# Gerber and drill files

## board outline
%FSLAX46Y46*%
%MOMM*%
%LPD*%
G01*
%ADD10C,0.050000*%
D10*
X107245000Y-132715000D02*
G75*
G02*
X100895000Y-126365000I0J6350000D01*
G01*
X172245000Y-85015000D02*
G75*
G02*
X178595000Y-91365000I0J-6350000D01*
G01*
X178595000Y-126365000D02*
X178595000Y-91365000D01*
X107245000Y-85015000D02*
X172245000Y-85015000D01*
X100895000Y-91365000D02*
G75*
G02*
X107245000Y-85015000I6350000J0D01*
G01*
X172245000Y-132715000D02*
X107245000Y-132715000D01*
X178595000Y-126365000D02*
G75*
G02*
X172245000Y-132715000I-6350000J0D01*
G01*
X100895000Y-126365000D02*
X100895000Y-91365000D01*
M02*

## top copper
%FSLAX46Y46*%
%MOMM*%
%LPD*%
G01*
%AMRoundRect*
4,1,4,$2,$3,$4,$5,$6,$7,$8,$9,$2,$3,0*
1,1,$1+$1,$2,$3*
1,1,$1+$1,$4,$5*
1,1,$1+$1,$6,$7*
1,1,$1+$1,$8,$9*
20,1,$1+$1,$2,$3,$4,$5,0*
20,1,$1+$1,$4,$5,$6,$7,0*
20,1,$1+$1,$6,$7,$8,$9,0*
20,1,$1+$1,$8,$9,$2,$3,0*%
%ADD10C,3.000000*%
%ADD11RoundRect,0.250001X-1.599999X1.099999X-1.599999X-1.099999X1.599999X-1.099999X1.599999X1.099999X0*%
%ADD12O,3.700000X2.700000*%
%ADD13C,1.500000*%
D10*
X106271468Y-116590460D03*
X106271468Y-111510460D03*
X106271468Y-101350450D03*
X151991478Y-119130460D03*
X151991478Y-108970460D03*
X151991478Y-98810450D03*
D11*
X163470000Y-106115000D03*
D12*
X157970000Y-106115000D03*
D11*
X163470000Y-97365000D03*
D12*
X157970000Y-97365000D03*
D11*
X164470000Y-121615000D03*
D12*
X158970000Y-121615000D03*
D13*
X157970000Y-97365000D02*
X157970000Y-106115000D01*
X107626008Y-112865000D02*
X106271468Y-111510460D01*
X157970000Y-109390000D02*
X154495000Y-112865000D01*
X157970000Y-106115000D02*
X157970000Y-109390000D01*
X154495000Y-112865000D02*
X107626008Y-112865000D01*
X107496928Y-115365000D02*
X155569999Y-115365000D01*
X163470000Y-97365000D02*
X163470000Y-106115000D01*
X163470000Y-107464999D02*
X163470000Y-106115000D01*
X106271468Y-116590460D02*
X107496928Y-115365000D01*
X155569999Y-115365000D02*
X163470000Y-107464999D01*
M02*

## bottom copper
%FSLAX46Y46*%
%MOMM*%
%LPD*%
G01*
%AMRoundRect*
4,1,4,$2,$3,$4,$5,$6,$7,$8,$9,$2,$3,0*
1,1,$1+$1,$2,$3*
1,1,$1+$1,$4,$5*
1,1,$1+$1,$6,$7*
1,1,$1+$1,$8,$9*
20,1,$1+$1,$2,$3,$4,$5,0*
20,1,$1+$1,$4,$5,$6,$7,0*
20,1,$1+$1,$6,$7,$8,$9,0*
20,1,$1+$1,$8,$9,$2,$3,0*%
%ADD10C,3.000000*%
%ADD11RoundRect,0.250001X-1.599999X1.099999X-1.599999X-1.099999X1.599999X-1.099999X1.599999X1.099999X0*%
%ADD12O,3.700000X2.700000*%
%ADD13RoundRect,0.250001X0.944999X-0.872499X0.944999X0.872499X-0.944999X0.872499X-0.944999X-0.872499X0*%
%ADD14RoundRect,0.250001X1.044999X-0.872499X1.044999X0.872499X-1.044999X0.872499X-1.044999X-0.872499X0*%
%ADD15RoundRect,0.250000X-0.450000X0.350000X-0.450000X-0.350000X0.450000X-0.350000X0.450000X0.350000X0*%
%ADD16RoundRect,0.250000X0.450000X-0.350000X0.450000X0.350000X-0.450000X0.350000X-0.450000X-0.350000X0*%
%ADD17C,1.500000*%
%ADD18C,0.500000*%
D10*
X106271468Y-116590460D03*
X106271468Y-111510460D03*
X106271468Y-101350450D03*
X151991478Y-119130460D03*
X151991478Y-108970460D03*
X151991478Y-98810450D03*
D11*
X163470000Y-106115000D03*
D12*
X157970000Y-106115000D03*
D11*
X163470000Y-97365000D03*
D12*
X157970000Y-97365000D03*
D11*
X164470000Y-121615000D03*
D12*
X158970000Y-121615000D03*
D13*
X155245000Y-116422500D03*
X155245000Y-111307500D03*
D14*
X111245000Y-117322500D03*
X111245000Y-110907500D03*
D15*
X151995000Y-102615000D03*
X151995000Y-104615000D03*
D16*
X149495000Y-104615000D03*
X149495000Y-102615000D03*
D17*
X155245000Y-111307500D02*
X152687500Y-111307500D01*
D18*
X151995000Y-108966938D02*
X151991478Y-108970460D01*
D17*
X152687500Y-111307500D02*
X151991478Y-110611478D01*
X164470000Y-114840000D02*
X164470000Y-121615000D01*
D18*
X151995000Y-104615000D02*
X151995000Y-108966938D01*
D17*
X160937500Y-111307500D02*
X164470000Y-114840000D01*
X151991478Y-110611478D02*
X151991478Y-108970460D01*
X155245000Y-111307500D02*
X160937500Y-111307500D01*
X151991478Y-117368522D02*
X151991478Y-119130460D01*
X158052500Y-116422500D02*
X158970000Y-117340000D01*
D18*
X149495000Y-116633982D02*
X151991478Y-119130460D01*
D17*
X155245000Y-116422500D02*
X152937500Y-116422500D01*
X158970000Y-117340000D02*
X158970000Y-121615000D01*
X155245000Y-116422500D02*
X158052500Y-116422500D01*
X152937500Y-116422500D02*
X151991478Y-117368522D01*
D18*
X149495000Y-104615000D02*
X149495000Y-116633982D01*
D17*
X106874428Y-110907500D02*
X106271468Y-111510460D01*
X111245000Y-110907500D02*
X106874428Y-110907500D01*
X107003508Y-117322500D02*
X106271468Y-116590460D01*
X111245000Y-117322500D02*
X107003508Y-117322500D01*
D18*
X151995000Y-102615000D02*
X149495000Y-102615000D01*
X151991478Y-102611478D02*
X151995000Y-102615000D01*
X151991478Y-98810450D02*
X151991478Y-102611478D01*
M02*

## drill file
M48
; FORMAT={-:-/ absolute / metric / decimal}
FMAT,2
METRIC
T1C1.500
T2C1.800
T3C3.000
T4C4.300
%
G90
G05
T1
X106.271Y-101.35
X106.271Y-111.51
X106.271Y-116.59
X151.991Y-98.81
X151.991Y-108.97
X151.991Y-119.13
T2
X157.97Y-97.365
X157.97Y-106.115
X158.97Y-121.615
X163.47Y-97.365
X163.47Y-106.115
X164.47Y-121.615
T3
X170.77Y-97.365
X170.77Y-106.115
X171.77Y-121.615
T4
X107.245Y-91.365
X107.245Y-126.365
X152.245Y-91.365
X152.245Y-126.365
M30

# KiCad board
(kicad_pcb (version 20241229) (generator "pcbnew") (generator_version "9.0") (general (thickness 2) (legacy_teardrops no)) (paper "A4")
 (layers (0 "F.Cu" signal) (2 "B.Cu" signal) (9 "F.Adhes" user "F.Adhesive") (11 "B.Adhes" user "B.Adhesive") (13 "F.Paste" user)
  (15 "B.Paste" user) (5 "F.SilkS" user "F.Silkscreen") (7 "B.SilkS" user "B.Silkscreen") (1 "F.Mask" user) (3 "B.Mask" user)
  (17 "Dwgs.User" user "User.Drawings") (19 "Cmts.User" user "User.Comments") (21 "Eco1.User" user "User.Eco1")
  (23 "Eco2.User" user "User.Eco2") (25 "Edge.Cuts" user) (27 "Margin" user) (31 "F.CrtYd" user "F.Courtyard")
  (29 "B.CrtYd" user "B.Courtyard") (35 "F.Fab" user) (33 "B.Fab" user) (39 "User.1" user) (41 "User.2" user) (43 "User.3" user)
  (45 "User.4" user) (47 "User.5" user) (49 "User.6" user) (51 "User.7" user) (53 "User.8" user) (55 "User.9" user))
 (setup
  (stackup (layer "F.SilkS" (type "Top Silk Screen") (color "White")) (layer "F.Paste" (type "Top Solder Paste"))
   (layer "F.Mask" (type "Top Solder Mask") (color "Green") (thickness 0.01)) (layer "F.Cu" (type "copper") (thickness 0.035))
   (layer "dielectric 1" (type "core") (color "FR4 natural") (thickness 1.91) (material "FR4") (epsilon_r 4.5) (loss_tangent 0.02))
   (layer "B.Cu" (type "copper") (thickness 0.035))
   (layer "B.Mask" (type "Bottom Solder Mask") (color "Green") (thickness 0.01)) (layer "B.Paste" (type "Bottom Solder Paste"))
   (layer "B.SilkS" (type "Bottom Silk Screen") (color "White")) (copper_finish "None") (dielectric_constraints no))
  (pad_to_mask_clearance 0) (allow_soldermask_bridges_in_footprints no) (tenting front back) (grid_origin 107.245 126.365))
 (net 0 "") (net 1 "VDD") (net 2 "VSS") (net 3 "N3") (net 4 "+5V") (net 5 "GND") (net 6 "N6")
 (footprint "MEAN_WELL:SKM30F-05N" (layer "F.Cu") (at 129.185753 95.93234)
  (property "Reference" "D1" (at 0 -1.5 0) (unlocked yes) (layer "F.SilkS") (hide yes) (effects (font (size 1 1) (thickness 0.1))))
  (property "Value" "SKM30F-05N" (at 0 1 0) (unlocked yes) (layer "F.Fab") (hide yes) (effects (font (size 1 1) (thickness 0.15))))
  (pad "1" thru_hole circle (at -22.914285 20.65812 180) (size 3 3) (drill 1.5) (layers "*.Cu" "*.Mask") (remove_unused_layers no)
   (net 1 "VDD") (thermal_bridge_angle 90))
  (pad "2" thru_hole circle (at -22.914285 15.57812 180) (size 3 3) (drill 1.5) (layers "*.Cu" "*.Mask") (remove_unused_layers no)
   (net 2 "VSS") (thermal_bridge_angle 90))
  (pad "3" thru_hole circle (at -22.914285 5.41811 180) (size 3 3) (drill 1.5) (layers "*.Cu" "*.Mask") (remove_unused_layers no)
   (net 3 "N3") (thermal_bridge_angle 90))
  (pad "4" thru_hole circle (at 22.805725 23.19812 180) (size 3 3) (drill 1.5) (layers "*.Cu" "*.Mask") (remove_unused_layers no)
   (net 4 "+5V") (thermal_bridge_angle 90))
  (pad "5" thru_hole circle (at 22.805725 13.03812 180) (size 3 3) (drill 1.5) (layers "*.Cu" "*.Mask") (remove_unused_layers no)
   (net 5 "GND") (thermal_bridge_angle 90))
  (pad "6" thru_hole circle (at 22.805725 2.87811 180) (size 3 3) (drill 1.5) (layers "*.Cu" "*.Mask") (remove_unused_layers no)
   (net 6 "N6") (thermal_bridge_angle 90)))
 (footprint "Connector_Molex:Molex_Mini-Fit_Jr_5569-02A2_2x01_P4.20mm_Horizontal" (layer "F.Cu") (at 163.47 106.115 -90)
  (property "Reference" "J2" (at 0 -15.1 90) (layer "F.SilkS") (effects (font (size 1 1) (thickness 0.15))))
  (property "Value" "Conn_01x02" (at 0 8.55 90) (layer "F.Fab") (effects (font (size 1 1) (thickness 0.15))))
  (pad "" np_thru_hole circle (at 0 -7.3 270) (size 3 3) (drill 3) (layers "*.Cu" "*.Mask"))
  (pad "1" thru_hole roundrect (at 0 0 270) (size 2.7 3.7) (drill 1.8) (layers "*.Cu" "*.Mask") (remove_unused_layers no)
   (roundrect_rratio 0.092593) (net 1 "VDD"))
  (pad "2" thru_hole oval (at 0 5.5 270) (size 2.7 3.7) (drill 1.8) (layers "*.Cu" "*.Mask") (remove_unused_layers no) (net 2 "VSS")))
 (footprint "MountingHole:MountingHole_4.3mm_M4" (layer "F.Cu") (at 107.245 126.365)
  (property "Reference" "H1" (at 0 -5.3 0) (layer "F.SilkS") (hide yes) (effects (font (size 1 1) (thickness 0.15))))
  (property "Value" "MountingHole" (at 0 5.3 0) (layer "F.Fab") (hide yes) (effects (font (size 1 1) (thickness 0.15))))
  (pad "" np_thru_hole circle (at 0 0) (size 4.3 4.3) (drill 4.3) (layers "*.Cu" "*.Mask")))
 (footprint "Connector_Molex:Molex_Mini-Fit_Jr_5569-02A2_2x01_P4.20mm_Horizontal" (layer "F.Cu") (at 163.47 97.365 -90)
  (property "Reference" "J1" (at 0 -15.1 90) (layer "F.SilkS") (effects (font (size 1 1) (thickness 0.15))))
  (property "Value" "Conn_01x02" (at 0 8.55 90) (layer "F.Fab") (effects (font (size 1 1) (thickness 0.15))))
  (pad "" np_thru_hole circle (at 0 -7.3 270) (size 3 3) (drill 3) (layers "*.Cu" "*.Mask"))
  (pad "1" thru_hole roundrect (at 0 0 270) (size 2.7 3.7) (drill 1.8) (layers "*.Cu" "*.Mask") (remove_unused_layers no)
   (roundrect_rratio 0.092593) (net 1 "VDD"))
  (pad "2" thru_hole oval (at 0 5.5 270) (size 2.7 3.7) (drill 1.8) (layers "*.Cu" "*.Mask") (remove_unused_layers no) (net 2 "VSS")))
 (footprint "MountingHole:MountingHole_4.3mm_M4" (layer "F.Cu") (at 107.245 91.365)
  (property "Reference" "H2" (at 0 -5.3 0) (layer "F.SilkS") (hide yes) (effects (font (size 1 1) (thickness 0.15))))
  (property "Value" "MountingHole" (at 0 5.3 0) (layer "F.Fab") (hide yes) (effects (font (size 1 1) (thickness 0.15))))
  (pad "" np_thru_hole circle (at 0 0) (size 4.3 4.3) (drill 4.3) (layers "*.Cu" "*.Mask")))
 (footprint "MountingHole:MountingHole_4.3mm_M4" (layer "F.Cu") (at 152.245 91.365)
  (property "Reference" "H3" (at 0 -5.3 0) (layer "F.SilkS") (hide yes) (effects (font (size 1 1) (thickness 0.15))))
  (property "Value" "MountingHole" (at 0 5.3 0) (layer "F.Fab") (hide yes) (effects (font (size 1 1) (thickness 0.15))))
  (pad "" np_thru_hole circle (at 0 0) (size 4.3 4.3) (drill 4.3) (layers "*.Cu" "*.Mask")))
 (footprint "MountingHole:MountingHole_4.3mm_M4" (layer "F.Cu") (at 152.245 126.365)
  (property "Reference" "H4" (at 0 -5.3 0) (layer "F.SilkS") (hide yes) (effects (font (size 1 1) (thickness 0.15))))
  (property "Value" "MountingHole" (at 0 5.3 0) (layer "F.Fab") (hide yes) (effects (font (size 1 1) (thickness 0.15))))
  (pad "" np_thru_hole circle (at 0 0) (size 4.3 4.3) (drill 4.3) (layers "*.Cu" "*.Mask")))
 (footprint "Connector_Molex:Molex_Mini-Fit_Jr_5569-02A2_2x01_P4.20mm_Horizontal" (layer "F.Cu") (at 164.47 121.615 -90)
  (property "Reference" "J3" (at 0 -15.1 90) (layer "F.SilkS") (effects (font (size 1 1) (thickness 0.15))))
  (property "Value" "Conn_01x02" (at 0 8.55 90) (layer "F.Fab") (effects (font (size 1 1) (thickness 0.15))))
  (pad "" np_thru_hole circle (at 0 -7.3 270) (size 3 3) (drill 3) (layers "*.Cu" "*.Mask"))
  (pad "1" thru_hole roundrect (at 0 0 270) (size 2.7 3.7) (drill 1.8) (layers "*.Cu" "*.Mask") (remove_unused_layers no)
   (roundrect_rratio 0.092593) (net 5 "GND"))
  (pad "2" thru_hole oval (at 0 5.5 270) (size 2.7 3.7) (drill 1.8) (layers "*.Cu" "*.Mask") (remove_unused_layers no) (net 4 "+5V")))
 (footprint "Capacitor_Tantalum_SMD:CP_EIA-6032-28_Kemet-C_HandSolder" (layer "B.Cu") (at 155.245 113.865 90)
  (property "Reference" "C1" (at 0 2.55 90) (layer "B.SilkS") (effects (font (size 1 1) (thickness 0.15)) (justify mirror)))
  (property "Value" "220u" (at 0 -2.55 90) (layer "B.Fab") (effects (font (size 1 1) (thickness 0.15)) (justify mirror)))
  (pad "1" smd roundrect (at -2.5575 0 90) (size 2.245 2.39) (layers "B.Cu" "B.Mask" "B.Paste") (roundrect_rratio 0.111359) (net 4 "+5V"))
  (pad "2" smd roundrect (at 2.5575 0 90) (size 2.245 2.39) (layers "B.Cu" "B.Mask" "B.Paste") (roundrect_rratio 0.111359) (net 5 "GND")))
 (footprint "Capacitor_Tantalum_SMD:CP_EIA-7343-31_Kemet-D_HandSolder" (layer "B.Cu") (at 111.245 114.115 90)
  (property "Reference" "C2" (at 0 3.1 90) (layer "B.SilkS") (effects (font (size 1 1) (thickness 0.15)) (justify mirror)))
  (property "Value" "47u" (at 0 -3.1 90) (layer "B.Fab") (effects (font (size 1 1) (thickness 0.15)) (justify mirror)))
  (pad "1" smd roundrect (at -3.2075 0 90) (size 2.245 2.59) (layers "B.Cu" "B.Mask" "B.Paste") (roundrect_rratio 0.111359) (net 1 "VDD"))
  (pad "2" smd roundrect (at 3.2075 0 90) (size 2.245 2.59) (layers "B.Cu" "B.Mask" "B.Paste") (roundrect_rratio 0.111359) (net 2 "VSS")))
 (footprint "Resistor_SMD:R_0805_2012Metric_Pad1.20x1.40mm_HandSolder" (layer "B.Cu") (at 151.995 103.615 -90)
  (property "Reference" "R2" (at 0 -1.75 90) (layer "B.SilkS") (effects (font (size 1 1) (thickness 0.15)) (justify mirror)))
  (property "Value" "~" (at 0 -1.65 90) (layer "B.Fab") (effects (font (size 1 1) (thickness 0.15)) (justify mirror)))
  (pad "1" smd roundrect (at -1 0 270) (size 1.2 1.4) (layers "B.Cu" "B.Mask" "B.Paste") (roundrect_rratio 0.208333) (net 6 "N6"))
  (pad "2" smd roundrect (at 1 0 270) (size 1.2 1.4) (layers "B.Cu" "B.Mask" "B.Paste") (roundrect_rratio 0.208333) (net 5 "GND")))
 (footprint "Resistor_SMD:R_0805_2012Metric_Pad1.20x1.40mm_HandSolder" (layer "B.Cu") (at 149.495 103.615 90)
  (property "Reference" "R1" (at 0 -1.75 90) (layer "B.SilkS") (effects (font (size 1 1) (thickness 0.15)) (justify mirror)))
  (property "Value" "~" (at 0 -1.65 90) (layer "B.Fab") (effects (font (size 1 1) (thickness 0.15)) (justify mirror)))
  (pad "1" smd roundrect (at -1 0 90) (size 1.2 1.4) (layers "B.Cu" "B.Mask" "B.Paste") (roundrect_rratio 0.208333) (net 4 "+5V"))
  (pad "2" smd roundrect (at 1 0 90) (size 1.2 1.4) (layers "B.Cu" "B.Mask" "B.Paste") (roundrect_rratio 0.208333) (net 6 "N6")))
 (gr_arc (start 107.245 132.715) (mid 102.754872 130.855128) (end 100.895 126.365) (stroke (width 0.05) (type default)) (layer "Edge.Cuts"))
 (gr_arc (start 172.245 85.015) (mid 176.735128 86.874872) (end 178.595 91.365) (stroke (width 0.05) (type default)) (layer "Edge.Cuts"))
 (gr_line (start 178.595 126.365) (end 178.595 91.365) (stroke (width 0.05) (type default)) (layer "Edge.Cuts"))
 (gr_line (start 107.245 85.015) (end 172.245 85.015) (stroke (width 0.05) (type default)) (layer "Edge.Cuts"))
 (gr_arc (start 100.895 91.365) (mid 102.754872 86.874872) (end 107.245 85.015) (stroke (width 0.05) (type default)) (layer "Edge.Cuts"))
 (gr_line (start 172.245 132.715) (end 107.245 132.715) (stroke (width 0.05) (type default)) (layer "Edge.Cuts"))
 (gr_arc (start 178.595 126.365) (mid 176.735128 130.855128) (end 172.245 132.715) (stroke (width 0.05) (type default)) (layer "Edge.Cuts"))
 (gr_line (start 100.895 126.365) (end 100.895 91.365) (stroke (width 0.05) (type default)) (layer "Edge.Cuts"))
 (segment (start 155.245 111.3075) (end 152.6875 111.3075) (width 1.5) (layer "B.Cu") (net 5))
 (segment (start 151.995 108.966938) (end 151.991478 108.97046) (width 0.5) (layer "B.Cu") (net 5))
 (segment (start 152.6875 111.3075) (end 151.991478 110.611478) (width 1.5) (layer "B.Cu") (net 5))
 (segment (start 164.47 114.84) (end 164.47 121.615) (width 1.5) (layer "B.Cu") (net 5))
 (segment (start 151.995 104.615) (end 151.995 108.966938) (width 0.5) (layer "B.Cu") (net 5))
 (segment (start 160.9375 111.3075) (end 164.47 114.84) (width 1.5) (layer "B.Cu") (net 5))
 (segment (start 151.991478 110.611478) (end 151.991478 108.97046) (width 1.5) (layer "B.Cu") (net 5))
 (segment (start 155.245 111.3075) (end 160.9375 111.3075) (width 1.5) (layer "B.Cu") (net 5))
 (segment (start 151.991478 117.368522) (end 151.991478 119.13046) (width 1.5) (layer "B.Cu") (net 4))
 (segment (start 158.0525 116.4225) (end 158.97 117.34) (width 1.5) (layer "B.Cu") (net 4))
 (segment (start 149.495 116.633982) (end 151.991478 119.13046) (width 0.5) (layer "B.Cu") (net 4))
 (segment (start 155.245 116.4225) (end 152.9375 116.4225) (width 1.5) (layer "B.Cu") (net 4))
 (segment (start 158.97 117.34) (end 158.97 121.615) (width 1.5) (layer "B.Cu") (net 4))
 (segment (start 155.245 116.4225) (end 158.0525 116.4225) (width 1.5) (layer "B.Cu") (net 4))
 (segment (start 152.9375 116.4225) (end 151.991478 117.368522) (width 1.5) (layer "B.Cu") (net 4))
 (segment (start 149.495 104.615) (end 149.495 116.633982) (width 0.5) (layer "B.Cu") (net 4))
 (segment (start 157.97 97.365) (end 157.97 106.115) (width 1.5) (layer "F.Cu") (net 2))
 (segment (start 107.626008 112.865) (end 106.271468 111.51046) (width 1.5) (layer "F.Cu") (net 2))
 (segment (start 157.97 109.39) (end 154.495 112.865) (width 1.5) (layer "F.Cu") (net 2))
 (segment (start 157.97 106.115) (end 157.97 109.39) (width 1.5) (layer "F.Cu") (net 2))
 (segment (start 154.495 112.865) (end 107.626008 112.865) (width 1.5) (layer "F.Cu") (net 2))
 (segment (start 106.874428 110.9075) (end 106.271468 111.51046) (width 1.5) (layer "B.Cu") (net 2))
 (segment (start 111.245 110.9075) (end 106.874428 110.9075) (width 1.5) (layer "B.Cu") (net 2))
 (segment (start 107.496928 115.365) (end 155.569999 115.365) (width 1.5) (layer "F.Cu") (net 1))
 (segment (start 163.47 97.365) (end 163.47 106.115) (width 1.5) (layer "F.Cu") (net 1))
 (segment (start 163.47 107.464999) (end 163.47 106.115) (width 1.5) (layer "F.Cu") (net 1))
 (segment (start 106.271468 116.59046) (end 107.496928 115.365) (width 1.5) (layer "F.Cu") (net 1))
 (segment (start 155.569999 115.365) (end 163.47 107.464999) (width 1.5) (layer "F.Cu") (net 1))
 (segment (start 107.003508 117.3225) (end 106.271468 116.59046) (width 1.5) (layer "B.Cu") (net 1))
 (segment (start 111.245 117.3225) (end 107.003508 117.3225) (width 1.5) (layer "B.Cu") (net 1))
 (segment (start 151.995 102.615) (end 149.495 102.615) (width 0.5) (layer "B.Cu") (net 6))
 (segment (start 151.991478 102.611478) (end 151.995 102.615) (width 0.5) (layer "B.Cu") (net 6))
 (segment (start 151.991478 98.81045) (end 151.991478 102.611478) (width 0.5) (layer "B.Cu") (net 6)))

